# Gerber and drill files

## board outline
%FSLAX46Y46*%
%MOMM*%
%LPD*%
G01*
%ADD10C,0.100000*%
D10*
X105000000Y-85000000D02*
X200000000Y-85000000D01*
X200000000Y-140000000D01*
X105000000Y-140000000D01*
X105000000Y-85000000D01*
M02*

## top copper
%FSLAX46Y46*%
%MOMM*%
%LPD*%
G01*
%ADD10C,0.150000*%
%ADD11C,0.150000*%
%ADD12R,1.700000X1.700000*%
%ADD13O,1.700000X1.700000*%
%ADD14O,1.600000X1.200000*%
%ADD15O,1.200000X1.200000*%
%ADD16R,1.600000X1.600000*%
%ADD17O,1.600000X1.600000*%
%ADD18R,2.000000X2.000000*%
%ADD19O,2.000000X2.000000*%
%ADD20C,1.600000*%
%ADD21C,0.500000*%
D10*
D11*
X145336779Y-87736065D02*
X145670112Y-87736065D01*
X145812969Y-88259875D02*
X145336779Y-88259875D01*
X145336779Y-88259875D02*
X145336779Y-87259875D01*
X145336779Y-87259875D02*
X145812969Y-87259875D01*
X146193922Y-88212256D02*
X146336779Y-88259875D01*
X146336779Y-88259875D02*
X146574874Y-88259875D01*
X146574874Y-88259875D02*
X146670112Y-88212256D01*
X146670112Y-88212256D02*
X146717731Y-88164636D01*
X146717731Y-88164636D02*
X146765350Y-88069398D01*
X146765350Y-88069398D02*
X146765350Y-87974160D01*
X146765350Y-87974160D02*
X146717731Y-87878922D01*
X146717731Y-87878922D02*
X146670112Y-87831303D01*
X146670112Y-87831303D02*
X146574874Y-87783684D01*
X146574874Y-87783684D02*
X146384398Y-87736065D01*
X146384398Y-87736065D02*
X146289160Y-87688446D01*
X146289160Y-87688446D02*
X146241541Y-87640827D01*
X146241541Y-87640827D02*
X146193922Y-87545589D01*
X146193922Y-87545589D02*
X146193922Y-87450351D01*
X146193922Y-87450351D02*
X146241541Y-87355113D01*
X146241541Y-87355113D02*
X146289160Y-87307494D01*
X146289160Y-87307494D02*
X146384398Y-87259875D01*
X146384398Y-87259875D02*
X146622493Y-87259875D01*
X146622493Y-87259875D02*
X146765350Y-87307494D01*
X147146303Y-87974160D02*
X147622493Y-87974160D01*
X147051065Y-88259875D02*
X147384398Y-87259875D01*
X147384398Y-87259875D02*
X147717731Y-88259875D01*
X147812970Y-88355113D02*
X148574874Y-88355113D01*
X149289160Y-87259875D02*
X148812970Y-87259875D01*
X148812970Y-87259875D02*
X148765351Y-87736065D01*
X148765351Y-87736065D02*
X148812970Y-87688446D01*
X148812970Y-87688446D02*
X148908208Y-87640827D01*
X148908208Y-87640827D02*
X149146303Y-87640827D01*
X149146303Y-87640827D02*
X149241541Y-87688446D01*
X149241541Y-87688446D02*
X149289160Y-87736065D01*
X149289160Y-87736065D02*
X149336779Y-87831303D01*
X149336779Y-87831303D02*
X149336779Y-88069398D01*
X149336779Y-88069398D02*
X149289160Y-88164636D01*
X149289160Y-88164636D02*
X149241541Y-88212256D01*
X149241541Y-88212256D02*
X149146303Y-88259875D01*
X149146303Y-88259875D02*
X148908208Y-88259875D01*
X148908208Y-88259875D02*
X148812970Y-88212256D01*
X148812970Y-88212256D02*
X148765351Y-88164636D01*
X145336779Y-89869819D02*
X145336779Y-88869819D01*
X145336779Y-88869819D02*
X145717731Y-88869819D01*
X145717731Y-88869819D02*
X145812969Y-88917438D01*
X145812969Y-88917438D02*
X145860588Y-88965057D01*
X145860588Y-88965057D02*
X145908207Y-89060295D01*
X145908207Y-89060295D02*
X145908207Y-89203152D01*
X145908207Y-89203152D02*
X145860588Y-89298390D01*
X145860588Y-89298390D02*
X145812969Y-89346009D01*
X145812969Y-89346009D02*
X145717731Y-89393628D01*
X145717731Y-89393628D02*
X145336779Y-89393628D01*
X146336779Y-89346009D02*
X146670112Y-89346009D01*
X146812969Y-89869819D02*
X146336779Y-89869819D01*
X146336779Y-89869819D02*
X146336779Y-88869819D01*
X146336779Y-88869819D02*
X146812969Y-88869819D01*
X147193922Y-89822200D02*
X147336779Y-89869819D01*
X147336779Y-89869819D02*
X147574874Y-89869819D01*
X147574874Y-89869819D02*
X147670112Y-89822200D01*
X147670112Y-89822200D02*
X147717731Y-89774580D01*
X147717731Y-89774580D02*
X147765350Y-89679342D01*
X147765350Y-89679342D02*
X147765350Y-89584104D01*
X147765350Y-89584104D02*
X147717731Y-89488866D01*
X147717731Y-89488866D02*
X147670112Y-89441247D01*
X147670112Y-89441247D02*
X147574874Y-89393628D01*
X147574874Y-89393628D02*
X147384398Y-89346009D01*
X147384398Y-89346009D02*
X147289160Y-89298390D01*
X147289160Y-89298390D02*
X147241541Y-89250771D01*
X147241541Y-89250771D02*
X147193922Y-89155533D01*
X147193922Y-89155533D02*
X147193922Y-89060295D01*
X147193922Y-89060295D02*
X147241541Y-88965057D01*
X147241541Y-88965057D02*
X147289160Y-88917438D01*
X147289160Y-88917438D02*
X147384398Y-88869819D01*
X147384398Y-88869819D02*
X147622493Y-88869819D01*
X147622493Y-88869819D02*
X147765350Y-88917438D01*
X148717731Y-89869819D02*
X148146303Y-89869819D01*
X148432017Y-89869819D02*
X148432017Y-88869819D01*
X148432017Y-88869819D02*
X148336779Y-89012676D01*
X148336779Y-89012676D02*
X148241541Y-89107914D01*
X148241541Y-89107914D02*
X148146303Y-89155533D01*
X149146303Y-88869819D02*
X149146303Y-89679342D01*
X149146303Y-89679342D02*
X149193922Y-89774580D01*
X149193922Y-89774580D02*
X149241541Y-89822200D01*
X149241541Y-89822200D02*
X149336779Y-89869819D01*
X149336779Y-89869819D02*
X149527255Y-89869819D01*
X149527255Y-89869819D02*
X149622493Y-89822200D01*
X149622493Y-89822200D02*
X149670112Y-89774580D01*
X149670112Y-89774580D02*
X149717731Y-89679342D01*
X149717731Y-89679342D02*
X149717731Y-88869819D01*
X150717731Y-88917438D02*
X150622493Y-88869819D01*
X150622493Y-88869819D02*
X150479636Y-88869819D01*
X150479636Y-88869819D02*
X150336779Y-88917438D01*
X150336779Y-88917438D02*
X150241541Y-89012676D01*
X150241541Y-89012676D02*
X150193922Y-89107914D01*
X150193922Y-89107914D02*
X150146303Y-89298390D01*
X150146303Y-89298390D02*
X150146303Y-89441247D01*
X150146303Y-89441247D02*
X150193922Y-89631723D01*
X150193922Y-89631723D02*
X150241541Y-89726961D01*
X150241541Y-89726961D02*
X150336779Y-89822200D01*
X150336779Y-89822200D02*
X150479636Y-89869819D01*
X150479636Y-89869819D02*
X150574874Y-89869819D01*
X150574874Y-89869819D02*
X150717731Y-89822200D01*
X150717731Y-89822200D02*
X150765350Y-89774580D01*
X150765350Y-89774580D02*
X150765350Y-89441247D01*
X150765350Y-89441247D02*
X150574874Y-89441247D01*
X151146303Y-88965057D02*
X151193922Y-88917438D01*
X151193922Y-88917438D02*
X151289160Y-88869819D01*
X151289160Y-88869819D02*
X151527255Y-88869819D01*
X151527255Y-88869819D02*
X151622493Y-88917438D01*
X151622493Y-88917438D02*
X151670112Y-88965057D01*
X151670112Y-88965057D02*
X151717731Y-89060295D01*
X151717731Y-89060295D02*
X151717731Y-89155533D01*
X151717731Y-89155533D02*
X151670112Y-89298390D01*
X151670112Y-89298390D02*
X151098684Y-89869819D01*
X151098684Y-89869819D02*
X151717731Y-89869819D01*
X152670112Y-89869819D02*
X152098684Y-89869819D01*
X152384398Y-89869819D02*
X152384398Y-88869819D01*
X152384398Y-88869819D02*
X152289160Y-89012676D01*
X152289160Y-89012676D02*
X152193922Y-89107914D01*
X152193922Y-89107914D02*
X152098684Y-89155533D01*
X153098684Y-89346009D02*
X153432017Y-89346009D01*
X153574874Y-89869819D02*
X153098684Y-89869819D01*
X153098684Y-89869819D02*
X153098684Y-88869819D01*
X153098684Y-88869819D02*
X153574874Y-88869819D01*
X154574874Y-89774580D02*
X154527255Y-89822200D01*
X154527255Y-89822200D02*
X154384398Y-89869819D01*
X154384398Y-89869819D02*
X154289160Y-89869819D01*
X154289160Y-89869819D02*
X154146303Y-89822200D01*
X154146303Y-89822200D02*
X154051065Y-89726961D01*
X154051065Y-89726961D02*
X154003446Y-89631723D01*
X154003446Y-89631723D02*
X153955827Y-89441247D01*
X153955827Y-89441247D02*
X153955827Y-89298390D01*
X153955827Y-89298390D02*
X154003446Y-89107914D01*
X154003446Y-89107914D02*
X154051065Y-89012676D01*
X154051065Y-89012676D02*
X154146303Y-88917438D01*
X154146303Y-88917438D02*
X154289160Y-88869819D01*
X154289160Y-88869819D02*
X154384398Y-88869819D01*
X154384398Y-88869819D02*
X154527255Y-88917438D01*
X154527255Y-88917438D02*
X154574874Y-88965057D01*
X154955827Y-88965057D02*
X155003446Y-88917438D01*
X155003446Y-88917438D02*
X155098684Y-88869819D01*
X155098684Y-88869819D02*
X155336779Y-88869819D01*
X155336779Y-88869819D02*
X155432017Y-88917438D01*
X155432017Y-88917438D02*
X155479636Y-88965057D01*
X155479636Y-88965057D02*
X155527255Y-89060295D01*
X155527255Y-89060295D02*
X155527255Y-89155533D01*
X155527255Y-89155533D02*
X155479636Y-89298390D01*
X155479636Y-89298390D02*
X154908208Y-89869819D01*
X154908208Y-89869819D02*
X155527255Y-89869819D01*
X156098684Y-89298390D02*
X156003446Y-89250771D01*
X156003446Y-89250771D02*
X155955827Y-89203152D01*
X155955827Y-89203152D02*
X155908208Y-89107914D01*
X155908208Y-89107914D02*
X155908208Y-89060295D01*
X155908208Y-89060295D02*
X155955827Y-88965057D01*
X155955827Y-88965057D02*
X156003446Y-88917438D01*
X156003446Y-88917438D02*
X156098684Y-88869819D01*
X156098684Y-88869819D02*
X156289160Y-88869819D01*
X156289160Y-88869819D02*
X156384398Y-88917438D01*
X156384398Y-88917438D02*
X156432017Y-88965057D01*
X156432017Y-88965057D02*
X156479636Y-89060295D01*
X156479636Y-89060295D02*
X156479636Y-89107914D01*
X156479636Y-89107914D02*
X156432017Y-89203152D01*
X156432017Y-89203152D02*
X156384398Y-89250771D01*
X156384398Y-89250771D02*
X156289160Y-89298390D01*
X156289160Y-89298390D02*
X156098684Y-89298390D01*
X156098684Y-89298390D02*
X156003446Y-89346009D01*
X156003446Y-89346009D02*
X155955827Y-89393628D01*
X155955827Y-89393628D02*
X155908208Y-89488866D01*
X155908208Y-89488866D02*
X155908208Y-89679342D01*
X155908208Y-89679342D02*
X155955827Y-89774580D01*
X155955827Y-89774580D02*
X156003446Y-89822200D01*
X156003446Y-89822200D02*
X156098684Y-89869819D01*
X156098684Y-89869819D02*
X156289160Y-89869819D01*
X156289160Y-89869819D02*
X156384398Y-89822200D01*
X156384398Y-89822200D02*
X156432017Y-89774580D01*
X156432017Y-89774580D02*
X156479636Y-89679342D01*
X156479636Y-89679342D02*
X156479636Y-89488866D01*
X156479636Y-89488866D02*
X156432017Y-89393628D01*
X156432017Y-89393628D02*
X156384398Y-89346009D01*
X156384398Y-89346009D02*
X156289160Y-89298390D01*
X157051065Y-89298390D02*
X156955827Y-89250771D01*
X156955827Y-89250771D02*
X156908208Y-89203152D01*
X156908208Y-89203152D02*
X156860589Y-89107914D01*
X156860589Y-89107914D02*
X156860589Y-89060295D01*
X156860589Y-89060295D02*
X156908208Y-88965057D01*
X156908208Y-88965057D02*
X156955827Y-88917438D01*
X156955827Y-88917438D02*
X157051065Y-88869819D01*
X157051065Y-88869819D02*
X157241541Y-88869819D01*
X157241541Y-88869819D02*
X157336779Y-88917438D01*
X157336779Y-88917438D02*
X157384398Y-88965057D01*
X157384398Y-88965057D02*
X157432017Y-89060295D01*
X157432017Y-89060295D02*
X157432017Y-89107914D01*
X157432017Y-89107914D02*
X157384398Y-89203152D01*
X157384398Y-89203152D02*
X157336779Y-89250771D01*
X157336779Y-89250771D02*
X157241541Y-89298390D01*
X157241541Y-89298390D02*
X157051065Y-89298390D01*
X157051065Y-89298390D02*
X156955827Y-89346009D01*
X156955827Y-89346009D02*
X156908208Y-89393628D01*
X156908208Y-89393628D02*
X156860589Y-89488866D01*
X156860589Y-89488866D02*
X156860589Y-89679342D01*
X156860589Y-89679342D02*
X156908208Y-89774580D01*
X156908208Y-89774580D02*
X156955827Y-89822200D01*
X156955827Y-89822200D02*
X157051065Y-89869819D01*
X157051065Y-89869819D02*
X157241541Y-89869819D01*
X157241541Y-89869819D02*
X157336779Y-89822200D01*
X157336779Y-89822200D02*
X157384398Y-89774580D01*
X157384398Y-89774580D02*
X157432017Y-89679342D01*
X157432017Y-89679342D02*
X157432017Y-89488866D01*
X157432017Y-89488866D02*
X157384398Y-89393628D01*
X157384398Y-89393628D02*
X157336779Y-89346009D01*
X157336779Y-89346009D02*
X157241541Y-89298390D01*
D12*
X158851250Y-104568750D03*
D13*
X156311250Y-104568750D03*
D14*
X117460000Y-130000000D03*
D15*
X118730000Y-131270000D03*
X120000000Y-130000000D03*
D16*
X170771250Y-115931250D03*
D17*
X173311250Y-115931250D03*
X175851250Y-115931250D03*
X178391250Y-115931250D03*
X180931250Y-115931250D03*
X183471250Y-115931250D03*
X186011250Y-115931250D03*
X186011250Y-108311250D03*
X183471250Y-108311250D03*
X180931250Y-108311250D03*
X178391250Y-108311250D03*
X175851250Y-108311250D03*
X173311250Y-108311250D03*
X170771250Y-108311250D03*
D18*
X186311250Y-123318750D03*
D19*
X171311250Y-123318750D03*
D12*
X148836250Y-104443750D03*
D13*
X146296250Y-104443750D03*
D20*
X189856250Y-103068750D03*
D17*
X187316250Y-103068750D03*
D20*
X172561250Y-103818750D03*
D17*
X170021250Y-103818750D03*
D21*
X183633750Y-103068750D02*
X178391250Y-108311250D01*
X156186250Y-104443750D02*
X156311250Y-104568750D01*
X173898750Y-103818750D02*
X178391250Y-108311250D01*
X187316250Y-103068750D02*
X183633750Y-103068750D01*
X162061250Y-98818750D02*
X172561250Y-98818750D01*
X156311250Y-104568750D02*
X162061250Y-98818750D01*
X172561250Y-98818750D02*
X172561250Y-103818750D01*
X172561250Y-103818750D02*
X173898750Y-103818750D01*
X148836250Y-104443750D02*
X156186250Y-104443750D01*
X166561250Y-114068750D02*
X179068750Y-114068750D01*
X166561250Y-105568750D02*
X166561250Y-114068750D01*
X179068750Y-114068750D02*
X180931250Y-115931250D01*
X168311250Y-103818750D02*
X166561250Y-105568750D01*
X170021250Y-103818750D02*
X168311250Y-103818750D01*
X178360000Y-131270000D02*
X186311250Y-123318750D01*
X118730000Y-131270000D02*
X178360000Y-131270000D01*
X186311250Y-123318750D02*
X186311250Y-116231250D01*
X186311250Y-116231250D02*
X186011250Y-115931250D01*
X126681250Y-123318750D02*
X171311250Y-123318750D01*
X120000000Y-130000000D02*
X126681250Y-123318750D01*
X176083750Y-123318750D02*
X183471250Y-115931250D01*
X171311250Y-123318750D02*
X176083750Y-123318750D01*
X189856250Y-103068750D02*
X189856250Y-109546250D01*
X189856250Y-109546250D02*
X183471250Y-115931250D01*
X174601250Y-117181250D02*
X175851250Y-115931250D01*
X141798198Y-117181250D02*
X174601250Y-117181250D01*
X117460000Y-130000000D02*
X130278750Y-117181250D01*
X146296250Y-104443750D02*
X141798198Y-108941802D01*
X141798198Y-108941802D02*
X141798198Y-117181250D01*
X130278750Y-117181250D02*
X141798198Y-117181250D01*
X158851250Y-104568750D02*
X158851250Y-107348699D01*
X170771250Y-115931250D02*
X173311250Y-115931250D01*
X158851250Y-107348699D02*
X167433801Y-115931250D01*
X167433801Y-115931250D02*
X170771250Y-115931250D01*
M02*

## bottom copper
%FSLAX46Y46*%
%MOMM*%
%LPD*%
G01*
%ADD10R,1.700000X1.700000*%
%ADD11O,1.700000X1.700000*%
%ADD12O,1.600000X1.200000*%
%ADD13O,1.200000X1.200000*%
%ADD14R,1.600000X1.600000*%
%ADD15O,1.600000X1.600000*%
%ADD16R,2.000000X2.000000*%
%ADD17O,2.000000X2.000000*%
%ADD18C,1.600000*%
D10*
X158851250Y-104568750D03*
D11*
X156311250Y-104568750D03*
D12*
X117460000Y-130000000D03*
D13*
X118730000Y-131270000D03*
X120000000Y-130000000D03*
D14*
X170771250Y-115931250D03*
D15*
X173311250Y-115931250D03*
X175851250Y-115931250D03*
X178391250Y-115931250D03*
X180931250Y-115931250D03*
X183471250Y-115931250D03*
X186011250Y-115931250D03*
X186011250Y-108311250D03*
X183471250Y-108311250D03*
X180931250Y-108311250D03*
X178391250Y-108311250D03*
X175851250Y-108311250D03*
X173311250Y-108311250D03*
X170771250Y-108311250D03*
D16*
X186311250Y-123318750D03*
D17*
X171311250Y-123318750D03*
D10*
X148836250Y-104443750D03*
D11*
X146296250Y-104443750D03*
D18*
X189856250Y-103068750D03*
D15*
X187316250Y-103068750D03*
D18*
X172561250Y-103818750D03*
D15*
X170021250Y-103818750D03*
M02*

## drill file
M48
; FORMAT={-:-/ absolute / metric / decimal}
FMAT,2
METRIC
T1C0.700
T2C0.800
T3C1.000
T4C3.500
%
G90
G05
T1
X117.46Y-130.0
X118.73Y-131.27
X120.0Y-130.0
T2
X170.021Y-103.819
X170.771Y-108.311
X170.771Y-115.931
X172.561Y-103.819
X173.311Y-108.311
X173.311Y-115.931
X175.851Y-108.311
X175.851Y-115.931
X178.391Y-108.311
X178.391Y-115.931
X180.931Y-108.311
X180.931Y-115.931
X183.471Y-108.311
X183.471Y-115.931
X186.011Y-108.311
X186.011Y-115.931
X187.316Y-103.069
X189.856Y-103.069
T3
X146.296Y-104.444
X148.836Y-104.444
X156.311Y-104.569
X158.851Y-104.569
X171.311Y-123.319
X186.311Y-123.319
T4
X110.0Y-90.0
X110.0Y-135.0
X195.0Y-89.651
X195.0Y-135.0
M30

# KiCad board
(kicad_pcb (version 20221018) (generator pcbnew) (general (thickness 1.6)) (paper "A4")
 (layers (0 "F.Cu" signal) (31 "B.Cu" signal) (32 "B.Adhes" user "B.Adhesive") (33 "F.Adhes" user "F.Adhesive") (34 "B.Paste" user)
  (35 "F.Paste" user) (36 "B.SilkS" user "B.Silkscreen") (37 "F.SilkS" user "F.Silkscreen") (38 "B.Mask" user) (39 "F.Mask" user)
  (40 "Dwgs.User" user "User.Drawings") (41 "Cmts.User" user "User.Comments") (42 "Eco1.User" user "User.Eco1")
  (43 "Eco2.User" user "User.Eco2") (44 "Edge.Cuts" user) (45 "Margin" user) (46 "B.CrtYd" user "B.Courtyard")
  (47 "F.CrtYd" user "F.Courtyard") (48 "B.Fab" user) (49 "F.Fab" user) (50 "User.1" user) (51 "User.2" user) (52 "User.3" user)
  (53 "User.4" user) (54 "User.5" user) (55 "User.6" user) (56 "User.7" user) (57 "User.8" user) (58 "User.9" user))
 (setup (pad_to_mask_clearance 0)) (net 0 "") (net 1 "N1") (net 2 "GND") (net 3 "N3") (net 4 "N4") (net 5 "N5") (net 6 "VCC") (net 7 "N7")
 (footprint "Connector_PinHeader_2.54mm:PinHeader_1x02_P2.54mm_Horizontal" (layer "F.Cu") (at 158.85125 104.56875 -90)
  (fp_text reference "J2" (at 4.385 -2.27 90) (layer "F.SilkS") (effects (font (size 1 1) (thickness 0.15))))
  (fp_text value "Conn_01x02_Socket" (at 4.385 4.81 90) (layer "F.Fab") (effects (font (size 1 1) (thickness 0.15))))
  (pad "1" thru_hole rect (at 0 0 270) (size 1.7 1.7) (drill 1) (layers "*.Cu" "*.Mask") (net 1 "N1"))
  (pad "2" thru_hole oval (at 0 2.54 270) (size 1.7 1.7) (drill 1) (layers "*.Cu" "*.Mask") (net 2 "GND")))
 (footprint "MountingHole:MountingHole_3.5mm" (layer "F.Cu") (at 195 89.650552)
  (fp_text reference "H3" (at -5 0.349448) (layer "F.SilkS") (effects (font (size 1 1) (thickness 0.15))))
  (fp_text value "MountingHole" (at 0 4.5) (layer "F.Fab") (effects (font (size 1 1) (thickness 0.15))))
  (pad "" np_thru_hole circle (at 0 0) (size 3.5 3.5) (drill 3.5) (layers "*.Cu" "*.Mask")))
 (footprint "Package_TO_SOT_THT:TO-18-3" (layer "F.Cu") (at 117.46 130)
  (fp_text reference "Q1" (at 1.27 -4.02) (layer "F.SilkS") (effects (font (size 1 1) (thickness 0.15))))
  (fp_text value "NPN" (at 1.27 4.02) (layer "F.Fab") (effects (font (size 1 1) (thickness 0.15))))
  (pad "1" thru_hole oval (at 0 0) (size 1.6 1.2) (drill 0.7) (layers "*.Cu" "*.Mask") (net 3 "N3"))
  (pad "2" thru_hole oval (at 1.27 1.27) (size 1.2 1.2) (drill 0.7) (layers "*.Cu" "*.Mask") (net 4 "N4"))
  (pad "3" thru_hole oval (at 2.54 0) (size 1.2 1.2) (drill 0.7) (layers "*.Cu" "*.Mask") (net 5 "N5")))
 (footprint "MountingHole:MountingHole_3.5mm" (layer "F.Cu") (at 195 135)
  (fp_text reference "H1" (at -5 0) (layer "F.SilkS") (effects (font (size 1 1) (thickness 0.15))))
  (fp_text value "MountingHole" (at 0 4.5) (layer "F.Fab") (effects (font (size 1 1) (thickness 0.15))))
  (pad "" np_thru_hole circle (at 0 0) (size 3.5 3.5) (drill 3.5) (layers "*.Cu" "*.Mask")))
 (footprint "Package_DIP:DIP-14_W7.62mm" (layer "F.Cu") (at 170.77125 115.93125 90)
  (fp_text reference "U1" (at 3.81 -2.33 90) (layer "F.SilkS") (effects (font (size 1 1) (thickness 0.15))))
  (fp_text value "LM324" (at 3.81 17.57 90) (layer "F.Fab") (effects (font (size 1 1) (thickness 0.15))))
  (pad "1" thru_hole rect (at 0 0 90) (size 1.6 1.6) (drill 0.8) (layers "*.Cu" "*.Mask") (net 1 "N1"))
  (pad "2" thru_hole oval (at 0 2.54 90) (size 1.6 1.6) (drill 0.8) (layers "*.Cu" "*.Mask") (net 1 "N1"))
  (pad "3" thru_hole oval (at 0 5.08 90) (size 1.6 1.6) (drill 0.8) (layers "*.Cu" "*.Mask") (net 3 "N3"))
  (pad "4" thru_hole oval (at 0 7.62 90) (size 1.6 1.6) (drill 0.8) (layers "*.Cu" "*.Mask") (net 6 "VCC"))
  (pad "5" thru_hole oval (at 0 10.16 90) (size 1.6 1.6) (drill 0.8) (layers "*.Cu" "*.Mask") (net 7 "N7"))
  (pad "6" thru_hole oval (at 0 12.7 90) (size 1.6 1.6) (drill 0.8) (layers "*.Cu" "*.Mask") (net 5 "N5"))
  (pad "7" thru_hole oval (at 0 15.24 90) (size 1.6 1.6) (drill 0.8) (layers "*.Cu" "*.Mask") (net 4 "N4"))
  (pad "8" thru_hole oval (at 7.62 15.24 90) (size 1.6 1.6) (drill 0.8) (layers "*.Cu" "*.Mask"))
  (pad "9" thru_hole oval (at 7.62 12.7 90) (size 1.6 1.6) (drill 0.8) (layers "*.Cu" "*.Mask"))
  (pad "10" thru_hole oval (at 7.62 10.16 90) (size 1.6 1.6) (drill 0.8) (layers "*.Cu" "*.Mask"))
  (pad "11" thru_hole oval (at 7.62 7.62 90) (size 1.6 1.6) (drill 0.8) (layers "*.Cu" "*.Mask") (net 2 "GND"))
  (pad "12" thru_hole oval (at 7.62 5.08 90) (size 1.6 1.6) (drill 0.8) (layers "*.Cu" "*.Mask"))
  (pad "13" thru_hole oval (at 7.62 2.54 90) (size 1.6 1.6) (drill 0.8) (layers "*.Cu" "*.Mask"))
  (pad "14" thru_hole oval (at 7.62 0 90) (size 1.6 1.6) (drill 0.8) (layers "*.Cu" "*.Mask")))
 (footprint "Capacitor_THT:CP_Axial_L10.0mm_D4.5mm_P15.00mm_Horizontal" (layer "F.Cu") (at 186.31125 123.31875 180)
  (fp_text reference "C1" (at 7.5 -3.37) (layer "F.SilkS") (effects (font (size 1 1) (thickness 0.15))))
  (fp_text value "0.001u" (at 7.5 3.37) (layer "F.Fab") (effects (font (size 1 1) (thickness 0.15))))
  (pad "1" thru_hole rect (at 0 0 180) (size 2 2) (drill 1) (layers "*.Cu" "*.Mask") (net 4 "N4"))
  (pad "2" thru_hole oval (at 15 0 180) (size 2 2) (drill 1) (layers "*.Cu" "*.Mask") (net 5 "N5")))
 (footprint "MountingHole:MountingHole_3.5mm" (layer "F.Cu") (at 110 135)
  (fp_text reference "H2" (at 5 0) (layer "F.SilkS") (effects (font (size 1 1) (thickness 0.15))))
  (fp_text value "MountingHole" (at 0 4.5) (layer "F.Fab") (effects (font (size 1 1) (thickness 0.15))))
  (pad "" np_thru_hole circle (at 0 0) (size 3.5 3.5) (drill 3.5) (layers "*.Cu" "*.Mask")))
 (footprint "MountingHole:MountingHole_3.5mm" (layer "F.Cu") (at 110 90)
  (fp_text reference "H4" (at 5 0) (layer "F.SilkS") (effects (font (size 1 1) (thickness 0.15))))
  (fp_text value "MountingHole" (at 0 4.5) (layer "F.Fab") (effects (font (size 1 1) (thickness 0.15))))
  (pad "" np_thru_hole circle (at 0 0) (size 3.5 3.5) (drill 3.5) (layers "*.Cu" "*.Mask")))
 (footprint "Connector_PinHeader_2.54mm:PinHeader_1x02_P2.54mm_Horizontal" (layer "F.Cu") (at 148.83625 104.44375 -90)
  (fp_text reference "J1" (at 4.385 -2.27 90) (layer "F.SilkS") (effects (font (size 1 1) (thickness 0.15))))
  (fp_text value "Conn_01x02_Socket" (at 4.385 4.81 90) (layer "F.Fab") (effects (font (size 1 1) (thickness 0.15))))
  (pad "1" thru_hole rect (at 0 0 270) (size 1.7 1.7) (drill 1) (layers "*.Cu" "*.Mask") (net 2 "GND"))
  (pad "2" thru_hole oval (at 0 2.54 270) (size 1.7 1.7) (drill 1) (layers "*.Cu" "*.Mask") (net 3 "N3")))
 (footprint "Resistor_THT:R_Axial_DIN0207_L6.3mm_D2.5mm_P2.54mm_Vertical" (layer "F.Cu") (at 189.85625 103.06875 180)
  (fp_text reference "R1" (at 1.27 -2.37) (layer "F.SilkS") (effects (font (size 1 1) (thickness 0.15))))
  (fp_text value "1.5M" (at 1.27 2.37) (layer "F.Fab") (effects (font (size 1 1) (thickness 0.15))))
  (pad "1" thru_hole circle (at 0 0 180) (size 1.6 1.6) (drill 0.8) (layers "*.Cu" "*.Mask") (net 5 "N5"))
  (pad "2" thru_hole oval (at 2.54 0 180) (size 1.6 1.6) (drill 0.8) (layers "*.Cu" "*.Mask") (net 2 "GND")))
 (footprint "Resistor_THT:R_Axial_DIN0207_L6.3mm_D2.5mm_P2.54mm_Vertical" (layer "F.Cu") (at 172.56125 103.81875 180)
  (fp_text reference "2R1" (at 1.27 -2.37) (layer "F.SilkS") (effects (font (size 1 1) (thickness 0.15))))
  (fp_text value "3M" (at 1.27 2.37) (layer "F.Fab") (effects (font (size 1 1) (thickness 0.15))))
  (pad "1" thru_hole circle (at 0 0 180) (size 1.6 1.6) (drill 0.8) (layers "*.Cu" "*.Mask") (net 2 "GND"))
  (pad "2" thru_hole oval (at 2.54 0 180) (size 1.6 1.6) (drill 0.8) (layers "*.Cu" "*.Mask") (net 7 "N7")))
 (gr_poly (pts (xy 105 85) (xy 200 85) (xy 200 140) (xy 105 140)) (stroke (width 0.1) (type solid)) (fill none) (layer "Edge.Cuts"))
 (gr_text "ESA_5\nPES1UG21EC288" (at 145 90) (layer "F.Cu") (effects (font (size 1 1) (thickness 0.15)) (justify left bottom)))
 (segment (start 183.63375 103.06875) (end 178.39125 108.31125) (width 0.5) (layer "F.Cu") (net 2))
 (segment (start 156.18625 104.44375) (end 156.31125 104.56875) (width 0.5) (layer "F.Cu") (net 2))
 (segment (start 173.89875 103.81875) (end 178.39125 108.31125) (width 0.5) (layer "F.Cu") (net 2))
 (segment (start 187.31625 103.06875) (end 183.63375 103.06875) (width 0.5) (layer "F.Cu") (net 2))
 (segment (start 162.06125 98.81875) (end 172.56125 98.81875) (width 0.5) (layer "F.Cu") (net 2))
 (segment (start 156.31125 104.56875) (end 162.06125 98.81875) (width 0.5) (layer "F.Cu") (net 2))
 (segment (start 172.56125 98.81875) (end 172.56125 103.81875) (width 0.5) (layer "F.Cu") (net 2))
 (segment (start 172.56125 103.81875) (end 173.89875 103.81875) (width 0.5) (layer "F.Cu") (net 2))
 (segment (start 148.83625 104.44375) (end 156.18625 104.44375) (width 0.5) (layer "F.Cu") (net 2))
 (segment (start 166.56125 114.06875) (end 179.06875 114.06875) (width 0.5) (layer "F.Cu") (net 7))
 (segment (start 166.56125 105.56875) (end 166.56125 114.06875) (width 0.5) (layer "F.Cu") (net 7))
 (segment (start 179.06875 114.06875) (end 180.93125 115.93125) (width 0.5) (layer "F.Cu") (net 7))
 (segment (start 168.31125 103.81875) (end 166.56125 105.56875) (width 0.5) (layer "F.Cu") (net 7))
 (segment (start 170.02125 103.81875) (end 168.31125 103.81875) (width 0.5) (layer "F.Cu") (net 7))
 (segment (start 178.36 131.27) (end 186.31125 123.31875) (width 0.5) (layer "F.Cu") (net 4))
 (segment (start 118.73 131.27) (end 178.36 131.27) (width 0.5) (layer "F.Cu") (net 4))
 (segment (start 186.31125 123.31875) (end 186.31125 116.23125) (width 0.5) (layer "F.Cu") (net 4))
 (segment (start 186.31125 116.23125) (end 186.01125 115.93125) (width 0.5) (layer "F.Cu") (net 4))
 (segment (start 126.68125 123.31875) (end 171.31125 123.31875) (width 0.5) (layer "F.Cu") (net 5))
 (segment (start 120 130) (end 126.68125 123.31875) (width 0.5) (layer "F.Cu") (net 5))
 (segment (start 176.08375 123.31875) (end 183.47125 115.93125) (width 0.5) (layer "F.Cu") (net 5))
 (segment (start 171.31125 123.31875) (end 176.08375 123.31875) (width 0.5) (layer "F.Cu") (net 5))
 (segment (start 189.85625 103.06875) (end 189.85625 109.54625) (width 0.5) (layer "F.Cu") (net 5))
 (segment (start 189.85625 109.54625) (end 183.47125 115.93125) (width 0.5) (layer "F.Cu") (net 5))
 (segment (start 174.60125 117.18125) (end 175.85125 115.93125) (width 0.5) (layer "F.Cu") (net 3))
 (segment (start 141.798198 117.18125) (end 174.60125 117.18125) (width 0.5) (layer "F.Cu") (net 3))
 (segment (start 117.46 130) (end 130.27875 117.18125) (width 0.5) (layer "F.Cu") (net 3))
 (segment (start 146.29625 104.44375) (end 141.798198 108.941802) (width 0.5) (layer "F.Cu") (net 3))
 (segment (start 141.798198 108.941802) (end 141.798198 117.18125) (width 0.5) (layer "F.Cu") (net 3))
 (segment (start 130.27875 117.18125) (end 141.798198 117.18125) (width 0.5) (layer "F.Cu") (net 3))
 (segment (start 158.85125 104.56875) (end 158.85125 107.348699) (width 0.5) (layer "F.Cu") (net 1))
 (segment (start 170.77125 115.93125) (end 173.31125 115.93125) (width 0.5) (layer "F.Cu") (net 1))
 (segment (start 158.85125 107.348699) (end 167.433801 115.93125) (width 0.5) (layer "F.Cu") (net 1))
 (segment (start 167.433801 115.93125) (end 170.77125 115.93125) (width 0.5) (layer "F.Cu") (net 1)))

